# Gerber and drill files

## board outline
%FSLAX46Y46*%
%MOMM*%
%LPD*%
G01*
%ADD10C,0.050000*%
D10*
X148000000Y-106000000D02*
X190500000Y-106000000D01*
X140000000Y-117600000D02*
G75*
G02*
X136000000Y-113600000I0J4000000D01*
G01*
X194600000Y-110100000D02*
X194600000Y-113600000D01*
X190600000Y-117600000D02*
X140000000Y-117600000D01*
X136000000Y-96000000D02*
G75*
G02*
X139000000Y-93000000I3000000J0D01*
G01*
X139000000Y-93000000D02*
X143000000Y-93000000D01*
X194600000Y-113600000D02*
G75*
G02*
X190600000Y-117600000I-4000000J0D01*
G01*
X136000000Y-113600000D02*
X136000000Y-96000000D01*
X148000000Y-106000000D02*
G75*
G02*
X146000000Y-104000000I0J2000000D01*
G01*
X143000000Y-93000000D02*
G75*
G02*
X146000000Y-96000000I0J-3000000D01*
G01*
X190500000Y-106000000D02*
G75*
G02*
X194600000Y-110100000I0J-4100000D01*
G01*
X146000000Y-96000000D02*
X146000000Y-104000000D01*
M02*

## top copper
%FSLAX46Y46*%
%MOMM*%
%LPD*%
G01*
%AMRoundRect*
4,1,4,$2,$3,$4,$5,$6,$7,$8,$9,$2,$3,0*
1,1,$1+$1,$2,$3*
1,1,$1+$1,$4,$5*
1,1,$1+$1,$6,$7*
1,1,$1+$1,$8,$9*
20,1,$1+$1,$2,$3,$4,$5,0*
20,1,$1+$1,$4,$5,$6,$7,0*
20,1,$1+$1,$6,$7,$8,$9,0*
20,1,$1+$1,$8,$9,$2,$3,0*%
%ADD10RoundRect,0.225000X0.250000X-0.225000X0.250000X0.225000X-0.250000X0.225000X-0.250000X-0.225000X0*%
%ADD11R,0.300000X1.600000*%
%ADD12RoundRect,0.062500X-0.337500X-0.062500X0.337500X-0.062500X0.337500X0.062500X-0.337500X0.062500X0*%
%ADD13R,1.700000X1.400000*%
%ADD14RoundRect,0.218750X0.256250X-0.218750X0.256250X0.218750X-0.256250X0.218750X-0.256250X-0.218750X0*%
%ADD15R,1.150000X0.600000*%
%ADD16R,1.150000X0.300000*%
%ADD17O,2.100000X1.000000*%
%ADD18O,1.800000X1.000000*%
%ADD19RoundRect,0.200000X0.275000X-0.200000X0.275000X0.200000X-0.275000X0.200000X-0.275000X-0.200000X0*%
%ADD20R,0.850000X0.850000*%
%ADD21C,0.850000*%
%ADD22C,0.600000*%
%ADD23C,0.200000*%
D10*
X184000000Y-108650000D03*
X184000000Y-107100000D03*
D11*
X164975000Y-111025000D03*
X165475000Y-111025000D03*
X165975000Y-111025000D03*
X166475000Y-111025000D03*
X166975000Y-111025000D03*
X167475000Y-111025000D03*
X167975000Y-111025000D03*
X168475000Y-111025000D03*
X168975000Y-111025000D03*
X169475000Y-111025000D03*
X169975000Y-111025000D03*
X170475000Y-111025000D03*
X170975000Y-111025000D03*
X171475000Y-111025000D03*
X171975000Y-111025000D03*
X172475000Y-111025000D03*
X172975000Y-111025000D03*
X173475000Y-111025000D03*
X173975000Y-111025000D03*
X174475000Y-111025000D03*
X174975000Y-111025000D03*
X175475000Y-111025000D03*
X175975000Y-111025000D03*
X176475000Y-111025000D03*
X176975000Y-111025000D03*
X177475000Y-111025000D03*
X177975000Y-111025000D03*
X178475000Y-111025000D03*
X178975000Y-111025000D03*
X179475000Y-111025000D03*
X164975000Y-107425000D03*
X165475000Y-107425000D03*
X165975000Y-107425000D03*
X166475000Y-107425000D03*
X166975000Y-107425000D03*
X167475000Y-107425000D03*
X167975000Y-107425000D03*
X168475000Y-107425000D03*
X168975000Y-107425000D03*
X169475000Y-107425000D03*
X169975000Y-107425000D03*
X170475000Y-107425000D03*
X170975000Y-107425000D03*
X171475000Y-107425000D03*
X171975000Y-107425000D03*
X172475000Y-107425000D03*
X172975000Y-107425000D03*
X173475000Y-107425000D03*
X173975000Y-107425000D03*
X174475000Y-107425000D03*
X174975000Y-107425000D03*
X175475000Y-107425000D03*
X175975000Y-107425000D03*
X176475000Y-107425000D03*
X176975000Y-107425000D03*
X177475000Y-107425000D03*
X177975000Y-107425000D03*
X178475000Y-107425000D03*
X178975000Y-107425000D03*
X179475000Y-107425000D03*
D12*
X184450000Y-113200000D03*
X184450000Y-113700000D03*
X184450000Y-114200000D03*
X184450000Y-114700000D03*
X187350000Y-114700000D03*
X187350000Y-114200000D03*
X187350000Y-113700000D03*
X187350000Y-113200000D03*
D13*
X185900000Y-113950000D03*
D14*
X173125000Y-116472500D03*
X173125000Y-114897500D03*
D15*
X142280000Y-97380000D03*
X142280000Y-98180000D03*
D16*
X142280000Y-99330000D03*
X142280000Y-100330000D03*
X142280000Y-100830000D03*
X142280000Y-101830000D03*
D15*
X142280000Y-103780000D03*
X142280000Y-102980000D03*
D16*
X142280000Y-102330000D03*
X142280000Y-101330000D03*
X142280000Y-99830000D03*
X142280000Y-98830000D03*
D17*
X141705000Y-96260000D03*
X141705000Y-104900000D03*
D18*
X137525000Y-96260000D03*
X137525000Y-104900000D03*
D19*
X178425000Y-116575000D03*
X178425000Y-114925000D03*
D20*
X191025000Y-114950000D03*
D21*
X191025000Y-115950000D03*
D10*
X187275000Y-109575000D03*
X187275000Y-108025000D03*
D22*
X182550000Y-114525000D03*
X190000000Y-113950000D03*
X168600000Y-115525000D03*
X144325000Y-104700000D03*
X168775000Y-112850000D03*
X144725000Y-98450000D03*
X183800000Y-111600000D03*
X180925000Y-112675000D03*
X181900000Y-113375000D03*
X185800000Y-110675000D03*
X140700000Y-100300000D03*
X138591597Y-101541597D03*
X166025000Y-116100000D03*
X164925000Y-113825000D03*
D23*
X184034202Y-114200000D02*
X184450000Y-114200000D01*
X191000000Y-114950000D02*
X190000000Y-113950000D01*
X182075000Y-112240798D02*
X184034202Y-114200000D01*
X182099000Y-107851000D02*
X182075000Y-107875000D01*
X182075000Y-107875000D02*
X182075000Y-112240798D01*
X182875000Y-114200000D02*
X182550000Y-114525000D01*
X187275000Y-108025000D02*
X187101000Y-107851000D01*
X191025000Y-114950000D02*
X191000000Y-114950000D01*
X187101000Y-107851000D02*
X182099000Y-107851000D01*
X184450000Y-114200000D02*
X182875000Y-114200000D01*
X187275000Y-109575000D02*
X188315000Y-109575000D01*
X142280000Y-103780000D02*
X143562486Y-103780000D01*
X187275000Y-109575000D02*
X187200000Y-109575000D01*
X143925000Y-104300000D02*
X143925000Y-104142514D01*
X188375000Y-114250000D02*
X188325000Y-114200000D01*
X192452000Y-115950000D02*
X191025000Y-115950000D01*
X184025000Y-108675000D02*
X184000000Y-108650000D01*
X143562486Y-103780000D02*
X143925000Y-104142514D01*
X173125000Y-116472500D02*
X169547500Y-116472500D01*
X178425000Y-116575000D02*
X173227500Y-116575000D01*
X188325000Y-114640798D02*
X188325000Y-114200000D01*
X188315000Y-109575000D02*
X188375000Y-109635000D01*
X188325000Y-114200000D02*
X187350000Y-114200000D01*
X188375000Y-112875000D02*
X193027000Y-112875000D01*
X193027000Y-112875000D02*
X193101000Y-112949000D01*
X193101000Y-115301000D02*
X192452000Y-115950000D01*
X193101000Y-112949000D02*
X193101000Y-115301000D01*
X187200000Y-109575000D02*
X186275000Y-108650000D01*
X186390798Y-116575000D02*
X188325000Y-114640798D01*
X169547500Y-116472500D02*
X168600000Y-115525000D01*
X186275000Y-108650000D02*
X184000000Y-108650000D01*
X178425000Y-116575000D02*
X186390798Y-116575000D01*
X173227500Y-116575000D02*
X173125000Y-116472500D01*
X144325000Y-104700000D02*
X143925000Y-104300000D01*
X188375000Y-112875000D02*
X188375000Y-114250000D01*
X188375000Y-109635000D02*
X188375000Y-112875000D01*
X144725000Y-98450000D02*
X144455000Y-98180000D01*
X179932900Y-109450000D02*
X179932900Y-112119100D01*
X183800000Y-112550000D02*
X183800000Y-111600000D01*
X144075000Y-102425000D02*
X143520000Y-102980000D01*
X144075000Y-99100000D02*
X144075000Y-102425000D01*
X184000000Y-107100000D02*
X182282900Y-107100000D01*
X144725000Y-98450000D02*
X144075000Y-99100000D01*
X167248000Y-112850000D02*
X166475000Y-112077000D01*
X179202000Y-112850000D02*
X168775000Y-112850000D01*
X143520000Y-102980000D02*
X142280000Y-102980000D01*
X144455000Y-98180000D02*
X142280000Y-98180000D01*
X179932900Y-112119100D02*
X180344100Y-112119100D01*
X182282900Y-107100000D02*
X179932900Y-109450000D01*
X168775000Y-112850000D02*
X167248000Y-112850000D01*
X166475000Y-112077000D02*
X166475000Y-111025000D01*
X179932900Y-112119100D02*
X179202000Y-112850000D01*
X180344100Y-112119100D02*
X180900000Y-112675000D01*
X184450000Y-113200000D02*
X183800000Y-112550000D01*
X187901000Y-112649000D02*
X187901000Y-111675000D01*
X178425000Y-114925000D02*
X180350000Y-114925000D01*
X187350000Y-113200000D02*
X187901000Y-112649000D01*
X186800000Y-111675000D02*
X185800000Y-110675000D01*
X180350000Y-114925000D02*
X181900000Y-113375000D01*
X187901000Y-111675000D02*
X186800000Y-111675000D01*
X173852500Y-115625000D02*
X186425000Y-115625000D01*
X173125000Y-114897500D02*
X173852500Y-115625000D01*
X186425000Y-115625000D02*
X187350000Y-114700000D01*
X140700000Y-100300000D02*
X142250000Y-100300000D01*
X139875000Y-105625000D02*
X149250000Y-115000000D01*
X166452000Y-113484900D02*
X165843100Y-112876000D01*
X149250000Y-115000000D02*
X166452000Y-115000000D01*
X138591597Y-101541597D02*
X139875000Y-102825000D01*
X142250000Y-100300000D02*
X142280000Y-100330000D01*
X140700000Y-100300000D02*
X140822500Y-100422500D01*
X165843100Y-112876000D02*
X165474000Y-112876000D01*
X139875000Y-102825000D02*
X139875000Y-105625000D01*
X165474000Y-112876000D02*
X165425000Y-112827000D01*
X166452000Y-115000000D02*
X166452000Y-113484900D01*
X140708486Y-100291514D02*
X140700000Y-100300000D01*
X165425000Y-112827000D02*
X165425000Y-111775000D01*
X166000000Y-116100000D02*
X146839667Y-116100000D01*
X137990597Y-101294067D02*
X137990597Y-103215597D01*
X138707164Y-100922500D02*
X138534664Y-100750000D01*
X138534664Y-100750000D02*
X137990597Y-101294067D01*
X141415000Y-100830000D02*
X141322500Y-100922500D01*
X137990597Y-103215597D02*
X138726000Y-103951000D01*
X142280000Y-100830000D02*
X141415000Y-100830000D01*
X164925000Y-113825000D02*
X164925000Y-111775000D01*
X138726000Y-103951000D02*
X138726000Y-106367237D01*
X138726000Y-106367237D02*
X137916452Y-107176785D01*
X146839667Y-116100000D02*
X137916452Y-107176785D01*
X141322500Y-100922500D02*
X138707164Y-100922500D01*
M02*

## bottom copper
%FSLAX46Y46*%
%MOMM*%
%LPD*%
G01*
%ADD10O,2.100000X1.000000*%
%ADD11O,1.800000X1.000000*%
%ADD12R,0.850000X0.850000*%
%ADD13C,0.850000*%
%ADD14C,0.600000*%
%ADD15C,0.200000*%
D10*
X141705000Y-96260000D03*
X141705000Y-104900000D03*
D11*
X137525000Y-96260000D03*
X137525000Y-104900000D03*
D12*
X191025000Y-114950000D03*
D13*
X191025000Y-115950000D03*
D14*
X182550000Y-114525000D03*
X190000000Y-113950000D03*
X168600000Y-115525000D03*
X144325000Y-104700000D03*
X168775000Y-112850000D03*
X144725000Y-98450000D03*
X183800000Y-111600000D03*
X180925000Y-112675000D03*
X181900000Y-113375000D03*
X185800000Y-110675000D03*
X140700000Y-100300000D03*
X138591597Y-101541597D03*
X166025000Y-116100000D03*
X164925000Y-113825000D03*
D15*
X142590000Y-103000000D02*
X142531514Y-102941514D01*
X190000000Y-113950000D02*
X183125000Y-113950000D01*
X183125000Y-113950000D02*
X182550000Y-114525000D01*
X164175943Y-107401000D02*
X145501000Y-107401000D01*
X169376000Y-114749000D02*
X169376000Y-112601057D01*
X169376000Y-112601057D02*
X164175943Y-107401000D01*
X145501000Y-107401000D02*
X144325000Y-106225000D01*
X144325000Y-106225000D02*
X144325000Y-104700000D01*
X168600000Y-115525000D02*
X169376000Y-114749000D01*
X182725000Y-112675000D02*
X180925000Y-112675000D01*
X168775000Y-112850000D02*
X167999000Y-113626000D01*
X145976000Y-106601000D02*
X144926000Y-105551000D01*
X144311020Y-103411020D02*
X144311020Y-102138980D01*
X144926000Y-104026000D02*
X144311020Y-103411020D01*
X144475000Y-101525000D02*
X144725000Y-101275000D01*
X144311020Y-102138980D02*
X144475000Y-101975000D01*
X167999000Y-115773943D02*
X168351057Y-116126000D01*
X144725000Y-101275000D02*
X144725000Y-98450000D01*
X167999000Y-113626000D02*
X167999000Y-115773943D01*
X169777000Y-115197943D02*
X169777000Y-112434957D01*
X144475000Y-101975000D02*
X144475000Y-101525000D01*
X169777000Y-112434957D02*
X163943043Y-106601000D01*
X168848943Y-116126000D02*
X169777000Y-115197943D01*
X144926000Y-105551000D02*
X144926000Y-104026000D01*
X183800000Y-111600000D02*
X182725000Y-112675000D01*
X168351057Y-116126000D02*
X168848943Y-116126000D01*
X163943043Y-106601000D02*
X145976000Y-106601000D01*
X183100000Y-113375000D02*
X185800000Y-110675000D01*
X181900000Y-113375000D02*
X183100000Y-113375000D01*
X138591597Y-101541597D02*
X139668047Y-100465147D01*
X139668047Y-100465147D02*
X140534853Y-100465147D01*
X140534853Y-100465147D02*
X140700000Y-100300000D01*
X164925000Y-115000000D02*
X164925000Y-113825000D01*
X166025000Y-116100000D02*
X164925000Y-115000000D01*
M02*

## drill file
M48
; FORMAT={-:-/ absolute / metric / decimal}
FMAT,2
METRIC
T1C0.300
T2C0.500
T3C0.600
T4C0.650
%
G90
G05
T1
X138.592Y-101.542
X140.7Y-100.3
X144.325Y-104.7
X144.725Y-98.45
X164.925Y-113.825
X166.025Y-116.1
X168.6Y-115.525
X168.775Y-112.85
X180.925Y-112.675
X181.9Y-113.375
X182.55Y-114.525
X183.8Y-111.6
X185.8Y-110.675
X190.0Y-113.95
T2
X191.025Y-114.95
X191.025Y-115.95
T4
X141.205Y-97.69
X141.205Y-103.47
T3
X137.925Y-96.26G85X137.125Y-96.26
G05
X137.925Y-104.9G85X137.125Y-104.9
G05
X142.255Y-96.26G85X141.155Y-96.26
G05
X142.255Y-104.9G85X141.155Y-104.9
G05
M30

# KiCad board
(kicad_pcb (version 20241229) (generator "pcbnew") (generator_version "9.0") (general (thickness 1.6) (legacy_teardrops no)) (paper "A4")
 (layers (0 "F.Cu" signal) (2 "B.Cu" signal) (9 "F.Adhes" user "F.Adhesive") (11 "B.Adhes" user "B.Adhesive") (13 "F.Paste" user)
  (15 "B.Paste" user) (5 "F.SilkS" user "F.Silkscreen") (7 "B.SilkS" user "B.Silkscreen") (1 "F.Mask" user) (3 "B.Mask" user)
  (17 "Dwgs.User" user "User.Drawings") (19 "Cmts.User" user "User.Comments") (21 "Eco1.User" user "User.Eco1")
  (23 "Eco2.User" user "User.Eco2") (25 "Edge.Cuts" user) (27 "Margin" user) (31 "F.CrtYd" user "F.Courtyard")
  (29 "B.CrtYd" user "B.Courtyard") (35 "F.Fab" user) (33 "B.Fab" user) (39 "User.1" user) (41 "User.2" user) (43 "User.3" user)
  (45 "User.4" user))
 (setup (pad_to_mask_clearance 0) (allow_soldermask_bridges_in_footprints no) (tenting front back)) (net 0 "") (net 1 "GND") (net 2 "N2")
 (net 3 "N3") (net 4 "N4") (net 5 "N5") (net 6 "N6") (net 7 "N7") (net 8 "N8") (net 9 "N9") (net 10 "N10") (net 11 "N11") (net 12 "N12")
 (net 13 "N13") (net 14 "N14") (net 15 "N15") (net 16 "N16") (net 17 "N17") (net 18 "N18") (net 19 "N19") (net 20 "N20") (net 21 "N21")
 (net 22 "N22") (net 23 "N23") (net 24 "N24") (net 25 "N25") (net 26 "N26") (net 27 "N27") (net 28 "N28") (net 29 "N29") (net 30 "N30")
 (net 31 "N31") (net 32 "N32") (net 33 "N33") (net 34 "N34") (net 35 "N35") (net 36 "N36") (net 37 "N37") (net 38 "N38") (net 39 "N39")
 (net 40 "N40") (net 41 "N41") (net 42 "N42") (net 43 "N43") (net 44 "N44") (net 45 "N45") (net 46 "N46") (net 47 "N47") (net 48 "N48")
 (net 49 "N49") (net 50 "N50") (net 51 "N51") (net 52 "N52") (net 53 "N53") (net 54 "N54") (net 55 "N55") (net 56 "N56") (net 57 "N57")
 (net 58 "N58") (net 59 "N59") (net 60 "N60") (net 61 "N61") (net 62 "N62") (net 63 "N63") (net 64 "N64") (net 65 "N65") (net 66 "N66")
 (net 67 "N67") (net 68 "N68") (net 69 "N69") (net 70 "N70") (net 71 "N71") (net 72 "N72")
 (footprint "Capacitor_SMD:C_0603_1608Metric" (layer "F.Cu") (at 184 107.875 90)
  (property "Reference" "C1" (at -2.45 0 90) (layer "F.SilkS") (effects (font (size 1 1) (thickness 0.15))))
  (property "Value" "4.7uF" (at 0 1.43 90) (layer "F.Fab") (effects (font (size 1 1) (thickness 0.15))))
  (pad "1" smd roundrect (at -0.775 0 90) (size 0.9 0.95) (layers "F.Cu" "F.Mask" "F.Paste") (roundrect_rratio 0.25) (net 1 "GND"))
  (pad "2" smd roundrect (at 0.775 0 90) (size 0.9 0.95) (layers "F.Cu" "F.Mask" "F.Paste") (roundrect_rratio 0.25) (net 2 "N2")))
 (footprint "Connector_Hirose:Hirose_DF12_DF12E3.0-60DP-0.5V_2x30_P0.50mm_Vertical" (layer "F.Cu") (at 172.225 109.225)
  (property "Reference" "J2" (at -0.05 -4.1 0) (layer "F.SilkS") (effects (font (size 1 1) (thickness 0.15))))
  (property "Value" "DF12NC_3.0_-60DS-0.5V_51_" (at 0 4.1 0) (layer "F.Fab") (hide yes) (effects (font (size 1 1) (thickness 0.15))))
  (pad "" smd rect (at -7.25 -2) (size 0.28 1.2) (layers "F.Paste"))
  (pad "" smd rect (at -7.25 2) (size 0.28 1.2) (layers "F.Paste"))
  (pad "" smd rect (at -6.75 -2) (size 0.28 1.2) (layers "F.Paste"))
  (pad "" smd rect (at -6.75 2) (size 0.28 1.2) (layers "F.Paste"))
  (pad "" smd rect (at -6.25 -2) (size 0.28 1.2) (layers "F.Paste"))
  (pad "" smd rect (at -6.25 2) (size 0.28 1.2) (layers "F.Paste"))
  (pad "" smd rect (at -5.75 -2) (size 0.28 1.2) (layers "F.Paste"))
  (pad "" smd rect (at -5.75 2) (size 0.28 1.2) (layers "F.Paste"))
  (pad "" smd rect (at -5.25 -2) (size 0.28 1.2) (layers "F.Paste"))
  (pad "" smd rect (at -5.25 2) (size 0.28 1.2) (layers "F.Paste"))
  (pad "" smd rect (at -4.75 -2) (size 0.28 1.2) (layers "F.Paste"))
  (pad "" smd rect (at -4.75 2) (size 0.28 1.2) (layers "F.Paste"))
  (pad "" smd rect (at -4.25 -2) (size 0.28 1.2) (layers "F.Paste"))
  (pad "" smd rect (at -4.25 2) (size 0.28 1.2) (layers "F.Paste"))
  (pad "" smd rect (at -3.75 -2) (size 0.28 1.2) (layers "F.Paste"))
  (pad "" smd rect (at -3.75 2) (size 0.28 1.2) (layers "F.Paste"))
  (pad "" smd rect (at -3.25 -2) (size 0.28 1.2) (layers "F.Paste"))
  (pad "" smd rect (at -3.25 2) (size 0.28 1.2) (layers "F.Paste"))
  (pad "" smd rect (at -2.75 -2) (size 0.28 1.2) (layers "F.Paste"))
  (pad "" smd rect (at -2.75 2) (size 0.28 1.2) (layers "F.Paste"))
  (pad "" smd rect (at -2.25 -2) (size 0.28 1.2) (layers "F.Paste"))
  (pad "" smd rect (at -2.25 2) (size 0.28 1.2) (layers "F.Paste"))
  (pad "" smd rect (at -1.75 -2) (size 0.28 1.2) (layers "F.Paste"))
  (pad "" smd rect (at -1.75 2) (size 0.28 1.2) (layers "F.Paste"))
  (pad "" smd rect (at -1.25 -2) (size 0.28 1.2) (layers "F.Paste"))
  (pad "" smd rect (at -1.25 2) (size 0.28 1.2) (layers "F.Paste"))
  (pad "" smd rect (at -0.75 -2) (size 0.28 1.2) (layers "F.Paste"))
  (pad "" smd rect (at -0.75 2) (size 0.28 1.2) (layers "F.Paste"))
  (pad "" smd rect (at -0.25 -2) (size 0.28 1.2) (layers "F.Paste"))
  (pad "" smd rect (at -0.25 2) (size 0.28 1.2) (layers "F.Paste"))
  (pad "" smd rect (at 0.25 -2) (size 0.28 1.2) (layers "F.Paste"))
  (pad "" smd rect (at 0.25 2) (size 0.28 1.2) (layers "F.Paste"))
  (pad "" smd rect (at 0.75 -2) (size 0.28 1.2) (layers "F.Paste"))
  (pad "" smd rect (at 0.75 2) (size 0.28 1.2) (layers "F.Paste"))
  (pad "" smd rect (at 1.25 -2) (size 0.28 1.2) (layers "F.Paste"))
  (pad "" smd rect (at 1.25 2) (size 0.28 1.2) (layers "F.Paste"))
  (pad "" smd rect (at 1.75 -2) (size 0.28 1.2) (layers "F.Paste"))
  (pad "" smd rect (at 1.75 2) (size 0.28 1.2) (layers "F.Paste"))
  (pad "" smd rect (at 2.25 -2) (size 0.28 1.2) (layers "F.Paste"))
  (pad "" smd rect (at 2.25 2) (size 0.28 1.2) (layers "F.Paste"))
  (pad "" smd rect (at 2.75 -2) (size 0.28 1.2) (layers "F.Paste"))
  (pad "" smd rect (at 2.75 2) (size 0.28 1.2) (layers "F.Paste"))
  (pad "" smd rect (at 3.25 -2) (size 0.28 1.2) (layers "F.Paste"))
  (pad "" smd rect (at 3.25 2) (size 0.28 1.2) (layers "F.Paste"))
  (pad "" smd rect (at 3.75 -2) (size 0.28 1.2) (layers "F.Paste"))
  (pad "" smd rect (at 3.75 2) (size 0.28 1.2) (layers "F.Paste"))
  (pad "" smd rect (at 4.25 -2) (size 0.28 1.2) (layers "F.Paste"))
  (pad "" smd rect (at 4.25 2) (size 0.28 1.2) (layers "F.Paste"))
  (pad "" smd rect (at 4.75 -2) (size 0.28 1.2) (layers "F.Paste"))
  (pad "" smd rect (at 4.75 2) (size 0.28 1.2) (layers "F.Paste"))
  (pad "" smd rect (at 5.25 -2) (size 0.28 1.2) (layers "F.Paste"))
  (pad "" smd rect (at 5.25 2) (size 0.28 1.2) (layers "F.Paste"))
  (pad "" smd rect (at 5.75 -2) (size 0.28 1.2) (layers "F.Paste"))
  (pad "" smd rect (at 5.75 2) (size 0.28 1.2) (layers "F.Paste"))
  (pad "" smd rect (at 6.25 -2) (size 0.28 1.2) (layers "F.Paste"))
  (pad "" smd rect (at 6.25 2) (size 0.28 1.2) (layers "F.Paste"))
  (pad "" smd rect (at 6.75 -2) (size 0.28 1.2) (layers "F.Paste"))
  (pad "" smd rect (at 6.75 2) (size 0.28 1.2) (layers "F.Paste"))
  (pad "" smd rect (at 7.25 -2) (size 0.28 1.2) (layers "F.Paste"))
  (pad "" smd rect (at 7.25 2) (size 0.28 1.2) (layers "F.Paste"))
  (pad "1" smd rect (at -7.25 1.8) (size 0.3 1.6) (layers "F.Cu" "F.Mask") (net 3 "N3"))
  (pad "2" smd rect (at -6.75 1.8) (size 0.3 1.6) (layers "F.Cu" "F.Mask") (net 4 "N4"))
  (pad "3" smd rect (at -6.25 1.8) (size 0.3 1.6) (layers "F.Cu" "F.Mask") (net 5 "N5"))
  (pad "4" smd rect (at -5.75 1.8) (size 0.3 1.6) (layers "F.Cu" "F.Mask") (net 2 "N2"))
  (pad "5" smd rect (at -5.25 1.8) (size 0.3 1.6) (layers "F.Cu" "F.Mask") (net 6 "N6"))
  (pad "6" smd rect (at -4.75 1.8) (size 0.3 1.6) (layers "F.Cu" "F.Mask") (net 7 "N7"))
  (pad "7" smd rect (at -4.25 1.8) (size 0.3 1.6) (layers "F.Cu" "F.Mask") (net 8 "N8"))
  (pad "8" smd rect (at -3.75 1.8) (size 0.3 1.6) (layers "F.Cu" "F.Mask") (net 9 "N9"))
  (pad "9" smd rect (at -3.25 1.8) (size 0.3 1.6) (layers "F.Cu" "F.Mask") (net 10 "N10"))
  (pad "10" smd rect (at -2.75 1.8) (size 0.3 1.6) (layers "F.Cu" "F.Mask") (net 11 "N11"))
  (pad "11" smd rect (at -2.25 1.8) (size 0.3 1.6) (layers "F.Cu" "F.Mask") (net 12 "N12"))
  (pad "12" smd rect (at -1.75 1.8) (size 0.3 1.6) (layers "F.Cu" "F.Mask") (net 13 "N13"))
  (pad "13" smd rect (at -1.25 1.8) (size 0.3 1.6) (layers "F.Cu" "F.Mask") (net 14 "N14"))
  (pad "14" smd rect (at -0.75 1.8) (size 0.3 1.6) (layers "F.Cu" "F.Mask") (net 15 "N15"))
  (pad "15" smd rect (at -0.25 1.8) (size 0.3 1.6) (layers "F.Cu" "F.Mask") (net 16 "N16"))
  (pad "16" smd rect (at 0.25 1.8) (size 0.3 1.6) (layers "F.Cu" "F.Mask") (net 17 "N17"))
  (pad "17" smd rect (at 0.75 1.8) (size 0.3 1.6) (layers "F.Cu" "F.Mask") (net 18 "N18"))
  (pad "18" smd rect (at 1.25 1.8) (size 0.3 1.6) (layers "F.Cu" "F.Mask") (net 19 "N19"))
  (pad "19" smd rect (at 1.75 1.8) (size 0.3 1.6) (layers "F.Cu" "F.Mask") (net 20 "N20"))
  (pad "20" smd rect (at 2.25 1.8) (size 0.3 1.6) (layers "F.Cu" "F.Mask") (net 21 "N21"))
  (pad "21" smd rect (at 2.75 1.8) (size 0.3 1.6) (layers "F.Cu" "F.Mask") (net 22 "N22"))
  (pad "22" smd rect (at 3.25 1.8) (size 0.3 1.6) (layers "F.Cu" "F.Mask") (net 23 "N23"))
  (pad "23" smd rect (at 3.75 1.8) (size 0.3 1.6) (layers "F.Cu" "F.Mask") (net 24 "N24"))
  (pad "24" smd rect (at 4.25 1.8) (size 0.3 1.6) (layers "F.Cu" "F.Mask") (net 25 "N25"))
  (pad "25" smd rect (at 4.75 1.8) (size 0.3 1.6) (layers "F.Cu" "F.Mask") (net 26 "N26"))
  (pad "26" smd rect (at 5.25 1.8) (size 0.3 1.6) (layers "F.Cu" "F.Mask") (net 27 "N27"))
  (pad "27" smd rect (at 5.75 1.8) (size 0.3 1.6) (layers "F.Cu" "F.Mask") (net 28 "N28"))
  (pad "28" smd rect (at 6.25 1.8) (size 0.3 1.6) (layers "F.Cu" "F.Mask") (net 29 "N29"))
  (pad "29" smd rect (at 6.75 1.8) (size 0.3 1.6) (layers "F.Cu" "F.Mask") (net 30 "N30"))
  (pad "30" smd rect (at 7.25 1.8) (size 0.3 1.6) (layers "F.Cu" "F.Mask") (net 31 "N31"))
  (pad "31" smd rect (at -7.25 -1.8) (size 0.3 1.6) (layers "F.Cu" "F.Mask") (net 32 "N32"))
  (pad "32" smd rect (at -6.75 -1.8) (size 0.3 1.6) (layers "F.Cu" "F.Mask") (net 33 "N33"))
  (pad "33" smd rect (at -6.25 -1.8) (size 0.3 1.6) (layers "F.Cu" "F.Mask") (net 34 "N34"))
  (pad "34" smd rect (at -5.75 -1.8) (size 0.3 1.6) (layers "F.Cu" "F.Mask") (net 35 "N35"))
  (pad "35" smd rect (at -5.25 -1.8) (size 0.3 1.6) (layers "F.Cu" "F.Mask") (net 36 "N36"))
  (pad "36" smd rect (at -4.75 -1.8) (size 0.3 1.6) (layers "F.Cu" "F.Mask") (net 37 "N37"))
  (pad "37" smd rect (at -4.25 -1.8) (size 0.3 1.6) (layers "F.Cu" "F.Mask") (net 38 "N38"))
  (pad "38" smd rect (at -3.75 -1.8) (size 0.3 1.6) (layers "F.Cu" "F.Mask") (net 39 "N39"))
  (pad "39" smd rect (at -3.25 -1.8) (size 0.3 1.6) (layers "F.Cu" "F.Mask") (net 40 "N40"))
  (pad "40" smd rect (at -2.75 -1.8) (size 0.3 1.6) (layers "F.Cu" "F.Mask") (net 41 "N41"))
  (pad "41" smd rect (at -2.25 -1.8) (size 0.3 1.6) (layers "F.Cu" "F.Mask") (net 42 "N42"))
  (pad "42" smd rect (at -1.75 -1.8) (size 0.3 1.6) (layers "F.Cu" "F.Mask") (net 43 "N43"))
  (pad "43" smd rect (at -1.25 -1.8) (size 0.3 1.6) (layers "F.Cu" "F.Mask") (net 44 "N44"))
  (pad "44" smd rect (at -0.75 -1.8) (size 0.3 1.6) (layers "F.Cu" "F.Mask") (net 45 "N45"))
  (pad "45" smd rect (at -0.25 -1.8) (size 0.3 1.6) (layers "F.Cu" "F.Mask") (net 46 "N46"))
  (pad "46" smd rect (at 0.25 -1.8) (size 0.3 1.6) (layers "F.Cu" "F.Mask") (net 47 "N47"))
  (pad "47" smd rect (at 0.75 -1.8) (size 0.3 1.6) (layers "F.Cu" "F.Mask") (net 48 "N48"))
  (pad "48" smd rect (at 1.25 -1.8) (size 0.3 1.6) (layers "F.Cu" "F.Mask") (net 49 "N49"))
  (pad "49" smd rect (at 1.75 -1.8) (size 0.3 1.6) (layers "F.Cu" "F.Mask") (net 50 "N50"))
  (pad "50" smd rect (at 2.25 -1.8) (size 0.3 1.6) (layers "F.Cu" "F.Mask") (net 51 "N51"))
  (pad "51" smd rect (at 2.75 -1.8) (size 0.3 1.6) (layers "F.Cu" "F.Mask") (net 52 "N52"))
  (pad "52" smd rect (at 3.25 -1.8) (size 0.3 1.6) (layers "F.Cu" "F.Mask") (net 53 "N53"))
  (pad "53" smd rect (at 3.75 -1.8) (size 0.3 1.6) (layers "F.Cu" "F.Mask") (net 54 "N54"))
  (pad "54" smd rect (at 4.25 -1.8) (size 0.3 1.6) (layers "F.Cu" "F.Mask") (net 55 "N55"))
  (pad "55" smd rect (at 4.75 -1.8) (size 0.3 1.6) (layers "F.Cu" "F.Mask") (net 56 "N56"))
  (pad "56" smd rect (at 5.25 -1.8) (size 0.3 1.6) (layers "F.Cu" "F.Mask") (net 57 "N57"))
  (pad "57" smd rect (at 5.75 -1.8) (size 0.3 1.6) (layers "F.Cu" "F.Mask") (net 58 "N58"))
  (pad "58" smd rect (at 6.25 -1.8) (size 0.3 1.6) (layers "F.Cu" "F.Mask") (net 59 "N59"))
  (pad "59" smd rect (at 6.75 -1.8) (size 0.3 1.6) (layers "F.Cu" "F.Mask") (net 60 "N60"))
  (pad "60" smd rect (at 7.25 -1.8) (size 0.3 1.6) (layers "F.Cu" "F.Mask") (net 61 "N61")))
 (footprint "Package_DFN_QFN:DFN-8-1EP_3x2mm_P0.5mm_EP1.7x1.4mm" (layer "F.Cu") (at 185.9 113.95)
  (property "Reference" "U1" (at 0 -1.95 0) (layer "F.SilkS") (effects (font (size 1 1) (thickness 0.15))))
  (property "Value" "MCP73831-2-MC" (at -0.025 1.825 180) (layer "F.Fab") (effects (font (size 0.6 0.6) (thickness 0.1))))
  (pad "" smd roundrect (at -0.425 -0.35) (size 0.69 0.56) (layers "F.Paste") (roundrect_rratio 0.25))
  (pad "" smd roundrect (at -0.425 0.35) (size 0.69 0.56) (layers "F.Paste") (roundrect_rratio 0.25))
  (pad "" smd roundrect (at 0.425 -0.35) (size 0.69 0.56) (layers "F.Paste") (roundrect_rratio 0.25))
  (pad "" smd roundrect (at 0.425 0.35) (size 0.69 0.56) (layers "F.Paste") (roundrect_rratio 0.25))
  (pad "1" smd roundrect (at -1.45 -0.75) (size 0.8 0.25) (layers "F.Cu" "F.Mask" "F.Paste") (roundrect_rratio 0.25) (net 2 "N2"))
  (pad "2" smd roundrect (at -1.45 -0.25) (size 0.8 0.25) (layers "F.Cu" "F.Mask" "F.Paste") (roundrect_rratio 0.25) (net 2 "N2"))
  (pad "3" smd roundrect (at -1.45 0.25) (size 0.8 0.25) (layers "F.Cu" "F.Mask" "F.Paste") (roundrect_rratio 0.25) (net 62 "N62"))
  (pad "4" smd roundrect (at -1.45 0.75) (size 0.8 0.25) (layers "F.Cu" "F.Mask" "F.Paste") (roundrect_rratio 0.25) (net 62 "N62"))
  (pad "5" smd roundrect (at 1.45 0.75) (size 0.8 0.25) (layers "F.Cu" "F.Mask" "F.Paste") (roundrect_rratio 0.25) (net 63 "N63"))
  (pad "6" smd roundrect (at 1.45 0.25) (size 0.8 0.25) (layers "F.Cu" "F.Mask" "F.Paste") (roundrect_rratio 0.25) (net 1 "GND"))
  (pad "7" smd roundrect (at 1.45 -0.25) (size 0.8 0.25) (layers "F.Cu" "F.Mask" "F.Paste") (roundrect_rratio 0.25) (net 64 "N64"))
  (pad "8" smd roundrect (at 1.45 -0.75) (size 0.8 0.25) (layers "F.Cu" "F.Mask" "F.Paste") (roundrect_rratio 0.25) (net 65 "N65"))
  (pad "9" smd rect (at 0 0) (size 1.7 1.4) (layers "F.Cu" "F.Mask") (zone_connect 2)))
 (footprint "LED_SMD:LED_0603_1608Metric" (layer "F.Cu") (at 173.125 115.685 90)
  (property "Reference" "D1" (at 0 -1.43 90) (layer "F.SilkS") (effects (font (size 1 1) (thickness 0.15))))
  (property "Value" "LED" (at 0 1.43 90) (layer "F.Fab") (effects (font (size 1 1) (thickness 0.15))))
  (pad "1" smd roundrect (at -0.7875 0 90) (size 0.875 0.95) (layers "F.Cu" "F.Mask" "F.Paste") (roundrect_rratio 0.25) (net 1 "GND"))
  (pad "2" smd roundrect (at 0.7875 0 90) (size 0.875 0.95) (layers "F.Cu" "F.Mask" "F.Paste") (roundrect_rratio 0.25) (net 63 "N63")))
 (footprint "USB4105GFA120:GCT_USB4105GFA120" (layer "F.Cu") (at 137.525 100.58 -90)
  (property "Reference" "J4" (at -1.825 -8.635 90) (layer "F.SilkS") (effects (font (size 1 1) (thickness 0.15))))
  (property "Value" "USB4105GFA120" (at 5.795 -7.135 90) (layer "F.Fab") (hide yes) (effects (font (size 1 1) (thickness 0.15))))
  (pad "" np_thru_hole circle (at -2.89 -3.68 270) (size 0.65 0.65) (drill 0.65) (layers "*.Cu" "*.Mask"))
  (pad "" np_thru_hole circle (at 2.89 -3.68 270) (size 0.65 0.65) (drill 0.65) (layers "*.Cu" "*.Mask"))
  (pad "A1_B12" smd rect (at -3.2 -4.755 270) (size 0.6 1.15) (layers "F.Cu" "F.Mask" "F.Paste") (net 1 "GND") (solder_mask_margin 0.102))
  (pad "A4_B9" smd rect (at -2.4 -4.755 270) (size 0.6 1.15) (layers "F.Cu" "F.Mask" "F.Paste") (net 2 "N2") (solder_mask_margin 0.102))
  (pad "A5" smd rect (at -1.25 -4.755 270) (size 0.3 1.15) (layers "F.Cu" "F.Mask" "F.Paste") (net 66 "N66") (solder_mask_margin 0.102))
  (pad "A6" smd rect (at -0.25 -4.755 270) (size 0.3 1.15) (layers "F.Cu" "F.Mask" "F.Paste") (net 4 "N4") (solder_mask_margin 0.102))
  (pad "A7" smd rect (at 0.25 -4.755 270) (size 0.3 1.15) (layers "F.Cu" "F.Mask" "F.Paste") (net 3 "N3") (solder_mask_margin 0.102))
  (pad "A8" smd rect (at 1.25 -4.755 270) (size 0.3 1.15) (layers "F.Cu" "F.Mask" "F.Paste") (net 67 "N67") (solder_mask_margin 0.102))
  (pad "B1_A12" smd rect (at 3.2 -4.755 270) (size 0.6 1.15) (layers "F.Cu" "F.Mask" "F.Paste") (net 1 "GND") (solder_mask_margin 0.102))
  (pad "B4_A9" smd rect (at 2.4 -4.755 270) (size 0.6 1.15) (layers "F.Cu" "F.Mask" "F.Paste") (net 2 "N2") (solder_mask_margin 0.102))
  (pad "B5" smd rect (at 1.75 -4.755 270) (size 0.3 1.15) (layers "F.Cu" "F.Mask" "F.Paste") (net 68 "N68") (solder_mask_margin 0.102))
  (pad "B6" smd rect (at 0.75 -4.755 270) (size 0.3 1.15) (layers "F.Cu" "F.Mask" "F.Paste") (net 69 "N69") (solder_mask_margin 0.102))
  (pad "B7" smd rect (at -0.75 -4.755 270) (size 0.3 1.15) (layers "F.Cu" "F.Mask" "F.Paste") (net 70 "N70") (solder_mask_margin 0.102))
  (pad "B8" smd rect (at -1.75 -4.755 270) (size 0.3 1.15) (layers "F.Cu" "F.Mask" "F.Paste") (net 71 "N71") (solder_mask_margin 0.102))
  (pad "SH1" thru_hole oval (at -4.32 -4.18 270) (size 1 2.1) (drill oval 0.6 1.7) (layers "*.Cu" "*.Mask") (remove_unused_layers no)
   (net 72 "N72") (solder_mask_margin 0.102))
  (pad "SH2" thru_hole oval (at 4.32 -4.18 270) (size 1 2.1) (drill oval 0.6 1.7) (layers "*.Cu" "*.Mask") (remove_unused_layers no)
   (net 72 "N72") (solder_mask_margin 0.102))
  (pad "SH3" thru_hole oval (at -4.32 0 270) (size 1 1.8) (drill oval 0.6 1.4) (layers "*.Cu" "*.Mask") (remove_unused_layers no)
   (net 72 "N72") (solder_mask_margin 0.102))
  (pad "SH4" thru_hole oval (at 4.32 0 270) (size 1 1.8) (drill oval 0.6 1.4) (layers "*.Cu" "*.Mask") (remove_unused_layers no)
   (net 72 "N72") (solder_mask_margin 0.102)))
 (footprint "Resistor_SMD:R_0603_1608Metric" (layer "F.Cu") (at 178.425 115.75 90)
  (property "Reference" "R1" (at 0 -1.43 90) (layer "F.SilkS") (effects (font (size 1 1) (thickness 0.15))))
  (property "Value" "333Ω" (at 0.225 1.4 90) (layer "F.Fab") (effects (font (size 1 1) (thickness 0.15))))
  (pad "1" smd roundrect (at -0.825 0 90) (size 0.8 0.95) (layers "F.Cu" "F.Mask" "F.Paste") (roundrect_rratio 0.25) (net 1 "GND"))
  (pad "2" smd roundrect (at 0.825 0 90) (size 0.8 0.95) (layers "F.Cu" "F.Mask" "F.Paste") (roundrect_rratio 0.25) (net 65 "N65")))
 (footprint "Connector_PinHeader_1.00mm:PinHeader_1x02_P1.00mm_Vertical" (layer "F.Cu") (at 191.025 114.95)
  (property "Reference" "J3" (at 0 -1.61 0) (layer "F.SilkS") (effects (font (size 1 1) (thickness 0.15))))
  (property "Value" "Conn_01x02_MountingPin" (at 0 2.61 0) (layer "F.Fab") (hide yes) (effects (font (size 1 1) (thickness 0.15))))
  (pad "1" thru_hole rect (at 0 0) (size 0.85 0.85) (drill 0.5) (layers "*.Cu" "*.Mask") (remove_unused_layers no) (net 62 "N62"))
  (pad "2" thru_hole circle (at 0 1) (size 0.85 0.85) (drill 0.5) (layers "*.Cu" "*.Mask") (remove_unused_layers no) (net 1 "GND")))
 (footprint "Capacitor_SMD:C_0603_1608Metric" (layer "F.Cu") (at 187.275 108.8 90)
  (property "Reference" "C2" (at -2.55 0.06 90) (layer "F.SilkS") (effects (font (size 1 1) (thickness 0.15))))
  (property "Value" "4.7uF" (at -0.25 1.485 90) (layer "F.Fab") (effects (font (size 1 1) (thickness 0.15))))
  (pad "1" smd roundrect (at -0.775 0 90) (size 0.9 0.95) (layers "F.Cu" "F.Mask" "F.Paste") (roundrect_rratio 0.25) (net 1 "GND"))
  (pad "2" smd roundrect (at 0.775 0 90) (size 0.9 0.95) (layers "F.Cu" "F.Mask" "F.Paste") (roundrect_rratio 0.25) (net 62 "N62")))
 (gr_line (start 148 106) (end 190.5 106) (stroke (width 0.05) (type default)) (layer "Edge.Cuts"))
 (gr_arc (start 140 117.6) (mid 137.171573 116.428427) (end 136 113.6) (stroke (width 0.05) (type default)) (layer "Edge.Cuts"))
 (gr_line (start 194.6 110.1) (end 194.6 113.6) (stroke (width 0.05) (type solid)) (layer "Edge.Cuts"))
 (gr_line (start 190.6 117.6) (end 140 117.6) (stroke (width 0.05) (type default)) (layer "Edge.Cuts"))
 (gr_arc (start 136 96) (mid 136.87868 93.87868) (end 139 93) (stroke (width 0.05) (type default)) (layer "Edge.Cuts"))
 (gr_line (start 139 93) (end 143 93) (stroke (width 0.05) (type default)) (layer "Edge.Cuts"))
 (gr_arc (start 194.6 113.6) (mid 193.428427 116.428427) (end 190.6 117.6) (stroke (width 0.05) (type default)) (layer "Edge.Cuts"))
 (gr_line (start 136 113.6) (end 136 96) (stroke (width 0.05) (type default)) (layer "Edge.Cuts"))
 (gr_arc (start 148 106) (mid 146.585786 105.414214) (end 146 104) (stroke (width 0.05) (type default)) (layer "Edge.Cuts"))
 (gr_arc (start 143 93) (mid 145.12132 93.87868) (end 146 96) (stroke (width 0.05) (type default)) (layer "Edge.Cuts"))
 (gr_arc (start 190.5 106) (mid 193.399138 107.200862) (end 194.6 110.1) (stroke (width 0.05) (type default)) (layer "Edge.Cuts"))
 (gr_line (start 146 96) (end 146 104) (stroke (width 0.05) (type solid)) (layer "Edge.Cuts"))
 (segment (start 142.59 103) (end 142.531514 102.941514) (width 0.2) (layer "B.Cu") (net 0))
 (segment (start 184.034202 114.2) (end 184.45 114.2) (width 0.2) (layer "F.Cu") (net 62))
 (segment (start 191 114.95) (end 190 113.95) (width 0.2) (layer "F.Cu") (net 62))
 (segment (start 182.075 112.240798) (end 184.034202 114.2) (width 0.2) (layer "F.Cu") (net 62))
 (segment (start 182.099 107.851) (end 182.075 107.875) (width 0.2) (layer "F.Cu") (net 62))
 (segment (start 182.075 107.875) (end 182.075 112.240798) (width 0.2) (layer "F.Cu") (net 62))
 (segment (start 182.875 114.2) (end 182.55 114.525) (width 0.2) (layer "F.Cu") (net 62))
 (segment (start 187.275 108.025) (end 187.101 107.851) (width 0.2) (layer "F.Cu") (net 62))
 (segment (start 191.025 114.95) (end 191 114.95) (width 0.2) (layer "F.Cu") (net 62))
 (segment (start 187.101 107.851) (end 182.099 107.851) (width 0.2) (layer "F.Cu") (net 62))
 (segment (start 184.45 114.2) (end 182.875 114.2) (width 0.2) (layer "F.Cu") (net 62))
 (via (at 182.55 114.525) (size 0.6) (drill 0.3) (layers "F.Cu" "B.Cu") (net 62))
 (via (at 190 113.95) (size 0.6) (drill 0.3) (layers "F.Cu" "B.Cu") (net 62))
 (segment (start 190 113.95) (end 183.125 113.95) (width 0.2) (layer "B.Cu") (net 62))
 (segment (start 183.125 113.95) (end 182.55 114.525) (width 0.2) (layer "B.Cu") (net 62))
 (segment (start 187.275 109.575) (end 188.315 109.575) (width 0.2) (layer "F.Cu") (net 1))
 (segment (start 142.28 103.78) (end 143.562486 103.78) (width 0.2) (layer "F.Cu") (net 1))
 (segment (start 187.275 109.575) (end 187.2 109.575) (width 0.2) (layer "F.Cu") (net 1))
 (segment (start 143.925 104.3) (end 143.925 104.142514) (width 0.2) (layer "F.Cu") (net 1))
 (segment (start 188.375 114.25) (end 188.325 114.2) (width 0.2) (layer "F.Cu") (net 1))
 (segment (start 192.452 115.95) (end 191.025 115.95) (width 0.2) (layer "F.Cu") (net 1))
 (segment (start 184.025 108.675) (end 184 108.65) (width 0.2) (layer "F.Cu") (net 1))
 (segment (start 143.562486 103.78) (end 143.925 104.142514) (width 0.2) (layer "F.Cu") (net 1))
 (segment (start 173.125 116.4725) (end 169.5475 116.4725) (width 0.2) (layer "F.Cu") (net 1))
 (segment (start 178.425 116.575) (end 173.2275 116.575) (width 0.2) (layer "F.Cu") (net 1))
 (segment (start 188.325 114.640798) (end 188.325 114.2) (width 0.2) (layer "F.Cu") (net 1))
 (segment (start 188.315 109.575) (end 188.375 109.635) (width 0.2) (layer "F.Cu") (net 1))
 (segment (start 188.325 114.2) (end 187.35 114.2) (width 0.2) (layer "F.Cu") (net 1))
 (segment (start 188.375 112.875) (end 193.027 112.875) (width 0.2) (layer "F.Cu") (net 1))
 (segment (start 193.027 112.875) (end 193.101 112.949) (width 0.2) (layer "F.Cu") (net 1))
 (segment (start 193.101 115.301) (end 192.452 115.95) (width 0.2) (layer "F.Cu") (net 1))
 (segment (start 193.101 112.949) (end 193.101 115.301) (width 0.2) (layer "F.Cu") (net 1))
 (segment (start 187.2 109.575) (end 186.275 108.65) (width 0.2) (layer "F.Cu") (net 1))
 (segment (start 186.390798 116.575) (end 188.325 114.640798) (width 0.2) (layer "F.Cu") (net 1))
 (segment (start 169.5475 116.4725) (end 168.6 115.525) (width 0.2) (layer "F.Cu") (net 1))
 (segment (start 186.275 108.65) (end 184 108.65) (width 0.2) (layer "F.Cu") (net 1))
 (segment (start 178.425 116.575) (end 186.390798 116.575) (width 0.2) (layer "F.Cu") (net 1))
 (segment (start 173.2275 116.575) (end 173.125 116.4725) (width 0.2) (layer "F.Cu") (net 1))
 (segment (start 144.325 104.7) (end 143.925 104.3) (width 0.2) (layer "F.Cu") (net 1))
 (segment (start 188.375 112.875) (end 188.375 114.25) (width 0.2) (layer "F.Cu") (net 1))
 (segment (start 188.375 109.635) (end 188.375 112.875) (width 0.2) (layer "F.Cu") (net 1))
 (via (at 168.6 115.525) (size 0.6) (drill 0.3) (layers "F.Cu" "B.Cu") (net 1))
 (via (at 144.325 104.7) (size 0.6) (drill 0.3) (layers "F.Cu" "B.Cu") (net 1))
 (segment (start 164.175943 107.401) (end 145.501 107.401) (width 0.2) (layer "B.Cu") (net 1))
 (segment (start 169.376 114.749) (end 169.376 112.601057) (width 0.2) (layer "B.Cu") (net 1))
 (segment (start 169.376 112.601057) (end 164.175943 107.401) (width 0.2) (layer "B.Cu") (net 1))
 (segment (start 145.501 107.401) (end 144.325 106.225) (width 0.2) (layer "B.Cu") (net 1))
 (segment (start 144.325 106.225) (end 144.325 104.7) (width 0.2) (layer "B.Cu") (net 1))
 (segment (start 168.6 115.525) (end 169.376 114.749) (width 0.2) (layer "B.Cu") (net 1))
 (segment (start 144.725 98.45) (end 144.455 98.18) (width 0.2) (layer "F.Cu") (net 2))
 (segment (start 179.9329 109.45) (end 179.9329 112.1191) (width 0.2) (layer "F.Cu") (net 2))
 (segment (start 183.8 112.55) (end 183.8 111.6) (width 0.2) (layer "F.Cu") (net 2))
 (segment (start 144.075 102.425) (end 143.52 102.98) (width 0.2) (layer "F.Cu") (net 2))
 (segment (start 144.075 99.1) (end 144.075 102.425) (width 0.2) (layer "F.Cu") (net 2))
 (segment (start 184 107.1) (end 182.2829 107.1) (width 0.2) (layer "F.Cu") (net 2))
 (segment (start 144.725 98.45) (end 144.075 99.1) (width 0.2) (layer "F.Cu") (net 2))
 (segment (start 167.248 112.85) (end 166.475 112.077) (width 0.2) (layer "F.Cu") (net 2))
 (segment (start 179.202 112.85) (end 168.775 112.85) (width 0.2) (layer "F.Cu") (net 2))
 (segment (start 143.52 102.98) (end 142.28 102.98) (width 0.2) (layer "F.Cu") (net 2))
 (segment (start 144.455 98.18) (end 142.28 98.18) (width 0.2) (layer "F.Cu") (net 2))
 (segment (start 179.9329 112.1191) (end 180.3441 112.1191) (width 0.2) (layer "F.Cu") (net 2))
 (segment (start 182.2829 107.1) (end 179.9329 109.45) (width 0.2) (layer "F.Cu") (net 2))
 (segment (start 168.775 112.85) (end 167.248 112.85) (width 0.2) (layer "F.Cu") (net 2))
 (segment (start 166.475 112.077) (end 166.475 111.025) (width 0.2) (layer "F.Cu") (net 2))
 (segment (start 179.9329 112.1191) (end 179.202 112.85) (width 0.2) (layer "F.Cu") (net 2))
 (segment (start 180.3441 112.1191) (end 180.9 112.675) (width 0.2) (layer "F.Cu") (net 2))
 (segment (start 184.45 113.2) (end 183.8 112.55) (width 0.2) (layer "F.Cu") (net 2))
 (via (at 168.775 112.85) (size 0.6) (drill 0.3) (layers "F.Cu" "B.Cu") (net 2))
 (via (at 144.725 98.45) (size 0.6) (drill 0.3) (layers "F.Cu" "B.Cu") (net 2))
 (via (at 183.8 111.6) (size 0.6) (drill 0.3) (layers "F.Cu" "B.Cu") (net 2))
 (via (at 180.925 112.675) (size 0.6) (drill 0.3) (layers "F.Cu" "B.Cu") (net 2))
 (segment (start 182.725 112.675) (end 180.925 112.675) (width 0.2) (layer "B.Cu") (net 2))
 (segment (start 168.775 112.85) (end 167.999 113.626) (width 0.2) (layer "B.Cu") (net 2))
 (segment (start 145.976 106.601) (end 144.926 105.551) (width 0.2) (layer "B.Cu") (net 2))
 (segment (start 144.31102 103.41102) (end 144.31102 102.13898) (width 0.2) (layer "B.Cu") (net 2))
 (segment (start 144.926 104.026) (end 144.31102 103.41102) (width 0.2) (layer "B.Cu") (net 2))
 (segment (start 144.475 101.525) (end 144.725 101.275) (width 0.2) (layer "B.Cu") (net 2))
 (segment (start 144.31102 102.13898) (end 144.475 101.975) (width 0.2) (layer "B.Cu") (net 2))
 (segment (start 167.999 115.773943) (end 168.351057 116.126) (width 0.2) (layer "B.Cu") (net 2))
 (segment (start 144.725 101.275) (end 144.725 98.45) (width 0.2) (layer "B.Cu") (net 2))
 (segment (start 167.999 113.626) (end 167.999 115.773943) (width 0.2) (layer "B.Cu") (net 2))
 (segment (start 169.777 115.197943) (end 169.777 112.434957) (width 0.2) (layer "B.Cu") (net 2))
 (segment (start 144.475 101.975) (end 144.475 101.525) (width 0.2) (layer "B.Cu") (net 2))
 (segment (start 169.777 112.434957) (end 163.943043 106.601) (width 0.2) (layer "B.Cu") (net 2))
 (segment (start 168.848943 116.126) (end 169.777 115.197943) (width 0.2) (layer "B.Cu") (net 2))
 (segment (start 144.926 105.551) (end 144.926 104.026) (width 0.2) (layer "B.Cu") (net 2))
 (segment (start 183.8 111.6) (end 182.725 112.675) (width 0.2) (layer "B.Cu") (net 2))
 (segment (start 168.351057 116.126) (end 168.848943 116.126) (width 0.2) (layer "B.Cu") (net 2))
 (segment (start 163.943043 106.601) (end 145.976 106.601) (width 0.2) (layer "B.Cu") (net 2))
 (segment (start 187.901 112.649) (end 187.901 111.675) (width 0.2) (layer "F.Cu") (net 65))
 (segment (start 178.425 114.925) (end 180.35 114.925) (width 0.2) (layer "F.Cu") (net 65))
 (segment (start 187.35 113.2) (end 187.901 112.649) (width 0.2) (layer "F.Cu") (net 65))
 (segment (start 186.8 111.675) (end 185.8 110.675) (width 0.2) (layer "F.Cu") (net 65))
 (segment (start 180.35 114.925) (end 181.9 113.375) (width 0.2) (layer "F.Cu") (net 65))
 (segment (start 187.901 111.675) (end 186.8 111.675) (width 0.2) (layer "F.Cu") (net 65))
 (via (at 181.9 113.375) (size 0.6) (drill 0.3) (layers "F.Cu" "B.Cu") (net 65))
 (via (at 185.8 110.675) (size 0.6) (drill 0.3) (layers "F.Cu" "B.Cu") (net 65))
 (segment (start 183.1 113.375) (end 185.8 110.675) (width 0.2) (layer "B.Cu") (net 65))
 (segment (start 181.9 113.375) (end 183.1 113.375) (width 0.2) (layer "B.Cu") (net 65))
 (segment (start 173.8525 115.625) (end 186.425 115.625) (width 0.2) (layer "F.Cu") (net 63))
 (segment (start 173.125 114.8975) (end 173.8525 115.625) (width 0.2) (layer "F.Cu") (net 63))
 (segment (start 186.425 115.625) (end 187.35 114.7) (width 0.2) (layer "F.Cu") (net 63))
 (segment (start 140.7 100.3) (end 142.25 100.3) (width 0.2) (layer "F.Cu") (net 4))
 (segment (start 139.875 105.625) (end 149.25 115) (width 0.2) (layer "F.Cu") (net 4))
 (segment (start 166.452 113.4849) (end 165.8431 112.876) (width 0.2) (layer "F.Cu") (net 4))
 (segment (start 149.25 115) (end 166.452 115) (width 0.2) (layer "F.Cu") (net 4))
 (segment (start 138.591597 101.541597) (end 139.875 102.825) (width 0.2) (layer "F.Cu") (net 4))
 (segment (start 142.25 100.3) (end 142.28 100.33) (width 0.2) (layer "F.Cu") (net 4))
 (segment (start 140.7 100.3) (end 140.8225 100.4225) (width 0.2) (layer "F.Cu") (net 4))
 (segment (start 165.8431 112.876) (end 165.474 112.876) (width 0.2) (layer "F.Cu") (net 4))
 (segment (start 139.875 102.825) (end 139.875 105.625) (width 0.2) (layer "F.Cu") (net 4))
 (segment (start 165.474 112.876) (end 165.425 112.827) (width 0.2) (layer "F.Cu") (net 4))
 (segment (start 166.452 115) (end 166.452 113.4849) (width 0.2) (layer "F.Cu") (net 4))
 (segment (start 140.708486 100.291514) (end 140.7 100.3) (width 0.2) (layer "F.Cu") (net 4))
 (segment (start 165.425 112.827) (end 165.425 111.775) (width 0.2) (layer "F.Cu") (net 4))
 (via (at 140.7 100.3) (size 0.6) (drill 0.3) (layers "F.Cu" "B.Cu") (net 4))
 (via (at 138.591597 101.541597) (size 0.6) (drill 0.3) (layers "F.Cu" "B.Cu") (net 4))
 (segment (start 138.591597 101.541597) (end 139.668047 100.465147) (width 0.2) (layer "B.Cu") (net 4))
 (segment (start 139.668047 100.465147) (end 140.534853 100.465147) (width 0.2) (layer "B.Cu") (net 4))
 (segment (start 140.534853 100.465147) (end 140.7 100.3) (width 0.2) (layer "B.Cu") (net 4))
 (segment (start 166 116.1) (end 146.839667 116.1) (width 0.2) (layer "F.Cu") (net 3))
 (segment (start 137.990597 101.294067) (end 137.990597 103.215597) (width 0.2) (layer "F.Cu") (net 3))
 (segment (start 138.707164 100.9225) (end 138.534664 100.75) (width 0.2) (layer "F.Cu") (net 3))
 (segment (start 138.534664 100.75) (end 137.990597 101.294067) (width 0.2) (layer "F.Cu") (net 3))
 (segment (start 141.415 100.83) (end 141.3225 100.9225) (width 0.2) (layer "F.Cu") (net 3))
 (segment (start 137.990597 103.215597) (end 138.726 103.951) (width 0.2) (layer "F.Cu") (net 3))
 (segment (start 142.28 100.83) (end 141.415 100.83) (width 0.2) (layer "F.Cu") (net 3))
 (segment (start 164.925 113.825) (end 164.925 111.775) (width 0.2) (layer "F.Cu") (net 3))
 (segment (start 138.726 103.951) (end 138.726 106.367237) (width 0.2) (layer "F.Cu") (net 3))
 (segment (start 138.726 106.367237) (end 137.916452 107.176785) (width 0.2) (layer "F.Cu") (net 3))
 (segment (start 146.839667 116.1) (end 137.916452 107.176785) (width 0.2) (layer "F.Cu") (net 3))
 (segment (start 141.3225 100.9225) (end 138.707164 100.9225) (width 0.2) (layer "F.Cu") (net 3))
 (via (at 166.025 116.1) (size 0.6) (drill 0.3) (layers "F.Cu" "B.Cu") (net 3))
 (via (at 164.925 113.825) (size 0.6) (drill 0.3) (layers "F.Cu" "B.Cu") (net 3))
 (segment (start 164.925 115) (end 164.925 113.825) (width 0.2) (layer "B.Cu") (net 3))
 (segment (start 166.025 116.1) (end 164.925 115) (width 0.2) (layer "B.Cu") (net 3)))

